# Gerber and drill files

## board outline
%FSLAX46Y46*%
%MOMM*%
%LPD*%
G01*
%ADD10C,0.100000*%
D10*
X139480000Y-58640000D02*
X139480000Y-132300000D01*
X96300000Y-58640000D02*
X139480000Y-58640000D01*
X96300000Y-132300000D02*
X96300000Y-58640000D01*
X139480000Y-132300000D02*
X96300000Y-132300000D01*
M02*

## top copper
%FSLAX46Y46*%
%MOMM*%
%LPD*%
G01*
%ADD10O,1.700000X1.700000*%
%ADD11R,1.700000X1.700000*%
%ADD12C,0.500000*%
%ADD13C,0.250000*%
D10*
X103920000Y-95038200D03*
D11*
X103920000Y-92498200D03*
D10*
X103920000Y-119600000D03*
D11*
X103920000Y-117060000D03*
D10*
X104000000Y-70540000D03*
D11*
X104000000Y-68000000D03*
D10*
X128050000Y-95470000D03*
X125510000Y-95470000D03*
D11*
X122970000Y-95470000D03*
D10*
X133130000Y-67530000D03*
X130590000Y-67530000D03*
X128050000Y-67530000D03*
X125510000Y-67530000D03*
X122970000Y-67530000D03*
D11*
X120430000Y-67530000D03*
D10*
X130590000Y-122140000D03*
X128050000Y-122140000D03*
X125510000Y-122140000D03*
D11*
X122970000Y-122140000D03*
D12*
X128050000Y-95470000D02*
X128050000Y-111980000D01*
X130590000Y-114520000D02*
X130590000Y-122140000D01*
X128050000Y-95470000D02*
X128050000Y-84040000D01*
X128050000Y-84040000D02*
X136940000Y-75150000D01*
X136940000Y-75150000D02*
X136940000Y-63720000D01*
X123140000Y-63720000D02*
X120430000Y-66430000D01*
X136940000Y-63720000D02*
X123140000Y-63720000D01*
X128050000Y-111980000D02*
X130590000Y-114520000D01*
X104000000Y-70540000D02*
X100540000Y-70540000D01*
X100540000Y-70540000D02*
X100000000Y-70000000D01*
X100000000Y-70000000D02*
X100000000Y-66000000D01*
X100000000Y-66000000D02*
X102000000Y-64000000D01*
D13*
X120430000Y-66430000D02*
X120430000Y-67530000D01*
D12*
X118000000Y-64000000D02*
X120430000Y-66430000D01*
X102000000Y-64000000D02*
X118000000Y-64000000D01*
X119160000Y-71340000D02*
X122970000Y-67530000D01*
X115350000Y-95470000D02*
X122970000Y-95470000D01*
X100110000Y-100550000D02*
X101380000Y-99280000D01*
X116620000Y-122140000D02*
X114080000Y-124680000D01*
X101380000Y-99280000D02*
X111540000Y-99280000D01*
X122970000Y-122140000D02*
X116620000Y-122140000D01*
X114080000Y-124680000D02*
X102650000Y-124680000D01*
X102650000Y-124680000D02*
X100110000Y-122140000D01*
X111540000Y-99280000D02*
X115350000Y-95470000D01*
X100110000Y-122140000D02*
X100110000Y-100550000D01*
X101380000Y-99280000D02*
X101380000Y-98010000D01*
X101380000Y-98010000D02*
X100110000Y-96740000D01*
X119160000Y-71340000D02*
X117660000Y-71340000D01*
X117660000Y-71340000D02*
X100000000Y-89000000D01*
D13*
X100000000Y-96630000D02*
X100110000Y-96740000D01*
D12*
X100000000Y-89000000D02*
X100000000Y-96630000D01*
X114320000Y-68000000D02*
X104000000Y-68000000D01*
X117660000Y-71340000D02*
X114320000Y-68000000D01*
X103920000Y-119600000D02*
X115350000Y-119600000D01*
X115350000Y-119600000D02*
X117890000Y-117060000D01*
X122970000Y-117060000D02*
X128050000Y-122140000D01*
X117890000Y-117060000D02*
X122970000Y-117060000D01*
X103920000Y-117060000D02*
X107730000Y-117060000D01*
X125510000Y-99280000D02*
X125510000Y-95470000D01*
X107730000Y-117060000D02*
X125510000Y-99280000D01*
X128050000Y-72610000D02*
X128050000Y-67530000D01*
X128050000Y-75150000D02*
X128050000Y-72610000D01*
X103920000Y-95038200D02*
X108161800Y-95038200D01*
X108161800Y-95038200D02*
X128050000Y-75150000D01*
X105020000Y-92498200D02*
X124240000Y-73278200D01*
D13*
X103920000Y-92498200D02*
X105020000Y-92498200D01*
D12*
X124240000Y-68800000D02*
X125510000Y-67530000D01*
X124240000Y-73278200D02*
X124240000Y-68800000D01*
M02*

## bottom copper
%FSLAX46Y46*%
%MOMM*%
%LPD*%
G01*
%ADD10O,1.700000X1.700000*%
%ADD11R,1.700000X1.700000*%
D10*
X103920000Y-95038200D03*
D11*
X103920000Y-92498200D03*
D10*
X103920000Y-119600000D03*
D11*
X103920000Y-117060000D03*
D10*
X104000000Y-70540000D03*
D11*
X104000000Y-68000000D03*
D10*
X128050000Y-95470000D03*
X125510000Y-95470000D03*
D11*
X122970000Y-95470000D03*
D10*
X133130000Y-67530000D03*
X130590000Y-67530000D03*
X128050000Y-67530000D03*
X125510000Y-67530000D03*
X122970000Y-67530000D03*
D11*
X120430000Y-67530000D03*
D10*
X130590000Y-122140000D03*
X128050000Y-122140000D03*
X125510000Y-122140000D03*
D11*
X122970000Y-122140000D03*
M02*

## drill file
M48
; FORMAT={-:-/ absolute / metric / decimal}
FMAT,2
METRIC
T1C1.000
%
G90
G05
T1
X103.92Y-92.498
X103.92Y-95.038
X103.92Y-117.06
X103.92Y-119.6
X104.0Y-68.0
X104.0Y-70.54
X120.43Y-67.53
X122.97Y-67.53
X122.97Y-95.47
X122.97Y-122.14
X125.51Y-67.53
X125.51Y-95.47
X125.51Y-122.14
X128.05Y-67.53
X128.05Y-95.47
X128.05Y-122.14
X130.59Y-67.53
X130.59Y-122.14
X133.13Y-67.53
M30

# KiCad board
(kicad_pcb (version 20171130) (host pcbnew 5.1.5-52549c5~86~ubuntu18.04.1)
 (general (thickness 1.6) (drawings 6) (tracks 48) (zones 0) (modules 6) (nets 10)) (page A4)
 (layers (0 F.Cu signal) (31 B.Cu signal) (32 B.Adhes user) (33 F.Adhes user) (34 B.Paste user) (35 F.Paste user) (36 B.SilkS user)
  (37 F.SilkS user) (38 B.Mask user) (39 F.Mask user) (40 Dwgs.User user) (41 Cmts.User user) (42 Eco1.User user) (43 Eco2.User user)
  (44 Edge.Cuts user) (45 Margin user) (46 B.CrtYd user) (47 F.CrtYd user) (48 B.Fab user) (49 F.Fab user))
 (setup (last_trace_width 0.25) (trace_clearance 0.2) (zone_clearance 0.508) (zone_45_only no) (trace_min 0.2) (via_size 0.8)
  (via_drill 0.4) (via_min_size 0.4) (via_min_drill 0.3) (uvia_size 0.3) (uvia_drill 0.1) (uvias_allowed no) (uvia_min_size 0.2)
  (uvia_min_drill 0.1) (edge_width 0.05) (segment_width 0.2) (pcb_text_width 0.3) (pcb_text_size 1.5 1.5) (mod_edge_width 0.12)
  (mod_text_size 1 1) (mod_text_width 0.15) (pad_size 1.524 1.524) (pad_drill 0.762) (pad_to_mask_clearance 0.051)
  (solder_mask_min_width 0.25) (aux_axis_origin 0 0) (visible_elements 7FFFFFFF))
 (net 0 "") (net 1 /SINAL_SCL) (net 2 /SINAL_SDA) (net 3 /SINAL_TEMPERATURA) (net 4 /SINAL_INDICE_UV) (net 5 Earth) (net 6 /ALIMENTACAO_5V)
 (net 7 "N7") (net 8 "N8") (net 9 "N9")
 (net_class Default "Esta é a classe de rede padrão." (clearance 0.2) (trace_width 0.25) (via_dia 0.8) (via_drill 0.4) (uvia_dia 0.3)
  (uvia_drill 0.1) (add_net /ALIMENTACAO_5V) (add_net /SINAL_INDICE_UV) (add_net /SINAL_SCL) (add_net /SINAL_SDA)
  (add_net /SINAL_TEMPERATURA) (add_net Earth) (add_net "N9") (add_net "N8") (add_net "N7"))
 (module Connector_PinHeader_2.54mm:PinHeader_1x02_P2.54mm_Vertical (layer F.Cu) (at 103.92 92.4982)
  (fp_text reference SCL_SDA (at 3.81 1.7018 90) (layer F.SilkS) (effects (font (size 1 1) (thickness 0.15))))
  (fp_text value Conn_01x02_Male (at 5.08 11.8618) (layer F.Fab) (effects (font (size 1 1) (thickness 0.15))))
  (pad 2 thru_hole oval (at 0 2.54) (size 1.7 1.7) (drill 1) (layers *.Cu *.Mask) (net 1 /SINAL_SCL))
  (pad 1 thru_hole rect (at 0 0) (size 1.7 1.7) (drill 1) (layers *.Cu *.Mask) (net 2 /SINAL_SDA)))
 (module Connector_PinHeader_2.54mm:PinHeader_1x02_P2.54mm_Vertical (layer F.Cu) (at 103.92 117.06)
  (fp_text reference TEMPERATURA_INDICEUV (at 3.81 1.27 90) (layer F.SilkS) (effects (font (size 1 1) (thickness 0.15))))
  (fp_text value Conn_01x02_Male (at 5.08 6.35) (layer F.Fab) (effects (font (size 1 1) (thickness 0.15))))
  (pad 2 thru_hole oval (at 0 2.54) (size 1.7 1.7) (drill 1) (layers *.Cu *.Mask) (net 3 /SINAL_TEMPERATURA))
  (pad 1 thru_hole rect (at 0 0) (size 1.7 1.7) (drill 1) (layers *.Cu *.Mask) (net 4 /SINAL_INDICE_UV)))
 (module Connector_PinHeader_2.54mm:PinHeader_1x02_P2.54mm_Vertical (layer F.Cu) (at 104 68)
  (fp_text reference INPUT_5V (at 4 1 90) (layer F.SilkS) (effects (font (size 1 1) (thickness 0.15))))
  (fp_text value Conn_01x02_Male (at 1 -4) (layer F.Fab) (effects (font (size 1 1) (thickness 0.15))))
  (pad 2 thru_hole oval (at 0 2.54) (size 1.7 1.7) (drill 1) (layers *.Cu *.Mask) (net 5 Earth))
  (pad 1 thru_hole rect (at 0 0) (size 1.7 1.7) (drill 1) (layers *.Cu *.Mask) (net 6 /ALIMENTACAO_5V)))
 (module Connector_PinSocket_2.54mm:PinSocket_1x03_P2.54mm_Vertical (layer F.Cu) (at 122.97 95.47 90)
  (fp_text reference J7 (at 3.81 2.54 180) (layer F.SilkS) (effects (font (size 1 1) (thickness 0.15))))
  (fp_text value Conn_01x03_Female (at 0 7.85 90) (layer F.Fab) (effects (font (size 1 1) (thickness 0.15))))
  (pad 3 thru_hole oval (at 0 5.08 90) (size 1.7 1.7) (drill 1) (layers *.Cu *.Mask) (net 5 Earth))
  (pad 2 thru_hole oval (at 0 2.54 90) (size 1.7 1.7) (drill 1) (layers *.Cu *.Mask) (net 4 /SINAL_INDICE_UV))
  (pad 1 thru_hole rect (at 0 0 90) (size 1.7 1.7) (drill 1) (layers *.Cu *.Mask) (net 6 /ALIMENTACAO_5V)))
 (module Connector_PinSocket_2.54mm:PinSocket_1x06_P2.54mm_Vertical (layer F.Cu) (at 120.43 67.53 90)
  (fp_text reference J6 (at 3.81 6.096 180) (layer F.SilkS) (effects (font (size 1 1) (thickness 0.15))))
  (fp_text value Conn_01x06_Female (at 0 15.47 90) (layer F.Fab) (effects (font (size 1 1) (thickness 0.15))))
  (pad 6 thru_hole oval (at 0 12.7 90) (size 1.7 1.7) (drill 1) (layers *.Cu *.Mask) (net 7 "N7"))
  (pad 5 thru_hole oval (at 0 10.16 90) (size 1.7 1.7) (drill 1) (layers *.Cu *.Mask) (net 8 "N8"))
  (pad 4 thru_hole oval (at 0 7.62 90) (size 1.7 1.7) (drill 1) (layers *.Cu *.Mask) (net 1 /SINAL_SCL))
  (pad 3 thru_hole oval (at 0 5.08 90) (size 1.7 1.7) (drill 1) (layers *.Cu *.Mask) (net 2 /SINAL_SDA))
  (pad 2 thru_hole oval (at 0 2.54 90) (size 1.7 1.7) (drill 1) (layers *.Cu *.Mask) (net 6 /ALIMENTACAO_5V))
  (pad 1 thru_hole rect (at 0 0 90) (size 1.7 1.7) (drill 1) (layers *.Cu *.Mask) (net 5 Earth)))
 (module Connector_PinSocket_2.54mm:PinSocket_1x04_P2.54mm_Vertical (layer F.Cu) (at 122.97 122.14 90)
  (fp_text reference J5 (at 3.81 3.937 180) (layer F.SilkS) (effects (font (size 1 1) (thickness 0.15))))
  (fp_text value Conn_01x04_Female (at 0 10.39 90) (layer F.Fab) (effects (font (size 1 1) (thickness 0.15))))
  (pad 4 thru_hole oval (at 0 7.62 90) (size 1.7 1.7) (drill 1) (layers *.Cu *.Mask) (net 5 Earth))
  (pad 3 thru_hole oval (at 0 5.08 90) (size 1.7 1.7) (drill 1) (layers *.Cu *.Mask) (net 3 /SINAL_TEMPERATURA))
  (pad 2 thru_hole oval (at 0 2.54 90) (size 1.7 1.7) (drill 1) (layers *.Cu *.Mask) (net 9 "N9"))
  (pad 1 thru_hole rect (at 0 0 90) (size 1.7 1.7) (drill 1) (layers *.Cu *.Mask) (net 6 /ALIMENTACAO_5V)))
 (gr_line (start 139.48 58.64) (end 139.48 132.3) (layer Edge.Cuts) (width 0.1))
 (gr_line (start 96.3 58.64) (end 139.48 58.64) (layer Edge.Cuts) (width 0.1))
 (gr_line (start 96.3 132.3) (end 96.3 58.64) (layer Edge.Cuts) (width 0.1))
 (gr_line (start 139.48 132.3) (end 96.3 132.3) (layer Edge.Cuts) (width 0.1))
 (segment (start 128.05 95.47) (end 128.05 111.98) (width 0.5) (layer F.Cu) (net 5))
 (segment (start 130.59 114.52) (end 130.59 122.14) (width 0.5) (layer F.Cu) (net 5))
 (segment (start 128.05 95.47) (end 128.05 84.04) (width 0.5) (layer F.Cu) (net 5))
 (segment (start 128.05 84.04) (end 136.94 75.15) (width 0.5) (layer F.Cu) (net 5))
 (segment (start 136.94 75.15) (end 136.94 63.72) (width 0.5) (layer F.Cu) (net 5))
 (segment (start 123.14 63.72) (end 120.43 66.43) (width 0.5) (layer F.Cu) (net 5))
 (segment (start 136.94 63.72) (end 123.14 63.72) (width 0.5) (layer F.Cu) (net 5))
 (segment (start 128.05 111.98) (end 130.59 114.52) (width 0.5) (layer F.Cu) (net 5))
 (segment (start 104 70.54) (end 100.54 70.54) (width 0.5) (layer F.Cu) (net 5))
 (segment (start 100.54 70.54) (end 100 70) (width 0.5) (layer F.Cu) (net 5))
 (segment (start 100 70) (end 100 66) (width 0.5) (layer F.Cu) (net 5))
 (segment (start 100 66) (end 102 64) (width 0.5) (layer F.Cu) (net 5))
 (segment (start 120.43 66.43) (end 120.43 67.53) (width 0.25) (layer F.Cu) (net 5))
 (segment (start 118 64) (end 120.43 66.43) (width 0.5) (layer F.Cu) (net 5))
 (segment (start 102 64) (end 118 64) (width 0.5) (layer F.Cu) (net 5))
 (segment (start 119.16 71.34) (end 122.97 67.53) (width 0.5) (layer F.Cu) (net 6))
 (segment (start 115.35 95.47) (end 122.97 95.47) (width 0.5) (layer F.Cu) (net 6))
 (segment (start 100.11 100.55) (end 101.38 99.28) (width 0.5) (layer F.Cu) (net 6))
 (segment (start 116.62 122.14) (end 114.08 124.68) (width 0.5) (layer F.Cu) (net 6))
 (segment (start 101.38 99.28) (end 111.54 99.28) (width 0.5) (layer F.Cu) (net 6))
 (segment (start 122.97 122.14) (end 116.62 122.14) (width 0.5) (layer F.Cu) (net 6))
 (segment (start 114.08 124.68) (end 102.65 124.68) (width 0.5) (layer F.Cu) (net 6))
 (segment (start 102.65 124.68) (end 100.11 122.14) (width 0.5) (layer F.Cu) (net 6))
 (segment (start 111.54 99.28) (end 115.35 95.47) (width 0.5) (layer F.Cu) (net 6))
 (segment (start 100.11 122.14) (end 100.11 100.55) (width 0.5) (layer F.Cu) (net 6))
 (segment (start 101.38 99.28) (end 101.38 98.01) (width 0.5) (layer F.Cu) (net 6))
 (segment (start 101.38 98.01) (end 100.11 96.74) (width 0.5) (layer F.Cu) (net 6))
 (segment (start 119.16 71.34) (end 117.66 71.34) (width 0.5) (layer F.Cu) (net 6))
 (segment (start 117.66 71.34) (end 100 89) (width 0.5) (layer F.Cu) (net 6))
 (segment (start 100 96.63) (end 100.11 96.74) (width 0.25) (layer F.Cu) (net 6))
 (segment (start 100 89) (end 100 96.63) (width 0.5) (layer F.Cu) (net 6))
 (segment (start 114.32 68) (end 104 68) (width 0.5) (layer F.Cu) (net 6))
 (segment (start 117.66 71.34) (end 114.32 68) (width 0.5) (layer F.Cu) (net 6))
 (segment (start 103.92 119.6) (end 115.35 119.6) (width 0.5) (layer F.Cu) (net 3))
 (segment (start 115.35 119.6) (end 117.89 117.06) (width 0.5) (layer F.Cu) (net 3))
 (segment (start 122.97 117.06) (end 128.05 122.14) (width 0.5) (layer F.Cu) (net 3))
 (segment (start 117.89 117.06) (end 122.97 117.06) (width 0.5) (layer F.Cu) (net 3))
 (segment (start 103.92 117.06) (end 107.73 117.06) (width 0.5) (layer F.Cu) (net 4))
 (segment (start 125.51 99.28) (end 125.51 95.47) (width 0.5) (layer F.Cu) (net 4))
 (segment (start 107.73 117.06) (end 125.51 99.28) (width 0.5) (layer F.Cu) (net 4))
 (segment (start 128.05 72.61) (end 128.05 67.53) (width 0.5) (layer F.Cu) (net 1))
 (segment (start 128.05 75.15) (end 128.05 72.61) (width 0.5) (layer F.Cu) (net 1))
 (segment (start 103.92 95.0382) (end 108.1618 95.0382) (width 0.5) (layer F.Cu) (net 1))
 (segment (start 108.1618 95.0382) (end 128.05 75.15) (width 0.5) (layer F.Cu) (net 1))
 (segment (start 105.02 92.4982) (end 124.24 73.2782) (width 0.5) (layer F.Cu) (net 2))
 (segment (start 103.92 92.4982) (end 105.02 92.4982) (width 0.25) (layer F.Cu) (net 2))
 (segment (start 124.24 68.8) (end 125.51 67.53) (width 0.5) (layer F.Cu) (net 2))
 (segment (start 124.24 73.2782) (end 124.24 68.8) (width 0.5) (layer F.Cu) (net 2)))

